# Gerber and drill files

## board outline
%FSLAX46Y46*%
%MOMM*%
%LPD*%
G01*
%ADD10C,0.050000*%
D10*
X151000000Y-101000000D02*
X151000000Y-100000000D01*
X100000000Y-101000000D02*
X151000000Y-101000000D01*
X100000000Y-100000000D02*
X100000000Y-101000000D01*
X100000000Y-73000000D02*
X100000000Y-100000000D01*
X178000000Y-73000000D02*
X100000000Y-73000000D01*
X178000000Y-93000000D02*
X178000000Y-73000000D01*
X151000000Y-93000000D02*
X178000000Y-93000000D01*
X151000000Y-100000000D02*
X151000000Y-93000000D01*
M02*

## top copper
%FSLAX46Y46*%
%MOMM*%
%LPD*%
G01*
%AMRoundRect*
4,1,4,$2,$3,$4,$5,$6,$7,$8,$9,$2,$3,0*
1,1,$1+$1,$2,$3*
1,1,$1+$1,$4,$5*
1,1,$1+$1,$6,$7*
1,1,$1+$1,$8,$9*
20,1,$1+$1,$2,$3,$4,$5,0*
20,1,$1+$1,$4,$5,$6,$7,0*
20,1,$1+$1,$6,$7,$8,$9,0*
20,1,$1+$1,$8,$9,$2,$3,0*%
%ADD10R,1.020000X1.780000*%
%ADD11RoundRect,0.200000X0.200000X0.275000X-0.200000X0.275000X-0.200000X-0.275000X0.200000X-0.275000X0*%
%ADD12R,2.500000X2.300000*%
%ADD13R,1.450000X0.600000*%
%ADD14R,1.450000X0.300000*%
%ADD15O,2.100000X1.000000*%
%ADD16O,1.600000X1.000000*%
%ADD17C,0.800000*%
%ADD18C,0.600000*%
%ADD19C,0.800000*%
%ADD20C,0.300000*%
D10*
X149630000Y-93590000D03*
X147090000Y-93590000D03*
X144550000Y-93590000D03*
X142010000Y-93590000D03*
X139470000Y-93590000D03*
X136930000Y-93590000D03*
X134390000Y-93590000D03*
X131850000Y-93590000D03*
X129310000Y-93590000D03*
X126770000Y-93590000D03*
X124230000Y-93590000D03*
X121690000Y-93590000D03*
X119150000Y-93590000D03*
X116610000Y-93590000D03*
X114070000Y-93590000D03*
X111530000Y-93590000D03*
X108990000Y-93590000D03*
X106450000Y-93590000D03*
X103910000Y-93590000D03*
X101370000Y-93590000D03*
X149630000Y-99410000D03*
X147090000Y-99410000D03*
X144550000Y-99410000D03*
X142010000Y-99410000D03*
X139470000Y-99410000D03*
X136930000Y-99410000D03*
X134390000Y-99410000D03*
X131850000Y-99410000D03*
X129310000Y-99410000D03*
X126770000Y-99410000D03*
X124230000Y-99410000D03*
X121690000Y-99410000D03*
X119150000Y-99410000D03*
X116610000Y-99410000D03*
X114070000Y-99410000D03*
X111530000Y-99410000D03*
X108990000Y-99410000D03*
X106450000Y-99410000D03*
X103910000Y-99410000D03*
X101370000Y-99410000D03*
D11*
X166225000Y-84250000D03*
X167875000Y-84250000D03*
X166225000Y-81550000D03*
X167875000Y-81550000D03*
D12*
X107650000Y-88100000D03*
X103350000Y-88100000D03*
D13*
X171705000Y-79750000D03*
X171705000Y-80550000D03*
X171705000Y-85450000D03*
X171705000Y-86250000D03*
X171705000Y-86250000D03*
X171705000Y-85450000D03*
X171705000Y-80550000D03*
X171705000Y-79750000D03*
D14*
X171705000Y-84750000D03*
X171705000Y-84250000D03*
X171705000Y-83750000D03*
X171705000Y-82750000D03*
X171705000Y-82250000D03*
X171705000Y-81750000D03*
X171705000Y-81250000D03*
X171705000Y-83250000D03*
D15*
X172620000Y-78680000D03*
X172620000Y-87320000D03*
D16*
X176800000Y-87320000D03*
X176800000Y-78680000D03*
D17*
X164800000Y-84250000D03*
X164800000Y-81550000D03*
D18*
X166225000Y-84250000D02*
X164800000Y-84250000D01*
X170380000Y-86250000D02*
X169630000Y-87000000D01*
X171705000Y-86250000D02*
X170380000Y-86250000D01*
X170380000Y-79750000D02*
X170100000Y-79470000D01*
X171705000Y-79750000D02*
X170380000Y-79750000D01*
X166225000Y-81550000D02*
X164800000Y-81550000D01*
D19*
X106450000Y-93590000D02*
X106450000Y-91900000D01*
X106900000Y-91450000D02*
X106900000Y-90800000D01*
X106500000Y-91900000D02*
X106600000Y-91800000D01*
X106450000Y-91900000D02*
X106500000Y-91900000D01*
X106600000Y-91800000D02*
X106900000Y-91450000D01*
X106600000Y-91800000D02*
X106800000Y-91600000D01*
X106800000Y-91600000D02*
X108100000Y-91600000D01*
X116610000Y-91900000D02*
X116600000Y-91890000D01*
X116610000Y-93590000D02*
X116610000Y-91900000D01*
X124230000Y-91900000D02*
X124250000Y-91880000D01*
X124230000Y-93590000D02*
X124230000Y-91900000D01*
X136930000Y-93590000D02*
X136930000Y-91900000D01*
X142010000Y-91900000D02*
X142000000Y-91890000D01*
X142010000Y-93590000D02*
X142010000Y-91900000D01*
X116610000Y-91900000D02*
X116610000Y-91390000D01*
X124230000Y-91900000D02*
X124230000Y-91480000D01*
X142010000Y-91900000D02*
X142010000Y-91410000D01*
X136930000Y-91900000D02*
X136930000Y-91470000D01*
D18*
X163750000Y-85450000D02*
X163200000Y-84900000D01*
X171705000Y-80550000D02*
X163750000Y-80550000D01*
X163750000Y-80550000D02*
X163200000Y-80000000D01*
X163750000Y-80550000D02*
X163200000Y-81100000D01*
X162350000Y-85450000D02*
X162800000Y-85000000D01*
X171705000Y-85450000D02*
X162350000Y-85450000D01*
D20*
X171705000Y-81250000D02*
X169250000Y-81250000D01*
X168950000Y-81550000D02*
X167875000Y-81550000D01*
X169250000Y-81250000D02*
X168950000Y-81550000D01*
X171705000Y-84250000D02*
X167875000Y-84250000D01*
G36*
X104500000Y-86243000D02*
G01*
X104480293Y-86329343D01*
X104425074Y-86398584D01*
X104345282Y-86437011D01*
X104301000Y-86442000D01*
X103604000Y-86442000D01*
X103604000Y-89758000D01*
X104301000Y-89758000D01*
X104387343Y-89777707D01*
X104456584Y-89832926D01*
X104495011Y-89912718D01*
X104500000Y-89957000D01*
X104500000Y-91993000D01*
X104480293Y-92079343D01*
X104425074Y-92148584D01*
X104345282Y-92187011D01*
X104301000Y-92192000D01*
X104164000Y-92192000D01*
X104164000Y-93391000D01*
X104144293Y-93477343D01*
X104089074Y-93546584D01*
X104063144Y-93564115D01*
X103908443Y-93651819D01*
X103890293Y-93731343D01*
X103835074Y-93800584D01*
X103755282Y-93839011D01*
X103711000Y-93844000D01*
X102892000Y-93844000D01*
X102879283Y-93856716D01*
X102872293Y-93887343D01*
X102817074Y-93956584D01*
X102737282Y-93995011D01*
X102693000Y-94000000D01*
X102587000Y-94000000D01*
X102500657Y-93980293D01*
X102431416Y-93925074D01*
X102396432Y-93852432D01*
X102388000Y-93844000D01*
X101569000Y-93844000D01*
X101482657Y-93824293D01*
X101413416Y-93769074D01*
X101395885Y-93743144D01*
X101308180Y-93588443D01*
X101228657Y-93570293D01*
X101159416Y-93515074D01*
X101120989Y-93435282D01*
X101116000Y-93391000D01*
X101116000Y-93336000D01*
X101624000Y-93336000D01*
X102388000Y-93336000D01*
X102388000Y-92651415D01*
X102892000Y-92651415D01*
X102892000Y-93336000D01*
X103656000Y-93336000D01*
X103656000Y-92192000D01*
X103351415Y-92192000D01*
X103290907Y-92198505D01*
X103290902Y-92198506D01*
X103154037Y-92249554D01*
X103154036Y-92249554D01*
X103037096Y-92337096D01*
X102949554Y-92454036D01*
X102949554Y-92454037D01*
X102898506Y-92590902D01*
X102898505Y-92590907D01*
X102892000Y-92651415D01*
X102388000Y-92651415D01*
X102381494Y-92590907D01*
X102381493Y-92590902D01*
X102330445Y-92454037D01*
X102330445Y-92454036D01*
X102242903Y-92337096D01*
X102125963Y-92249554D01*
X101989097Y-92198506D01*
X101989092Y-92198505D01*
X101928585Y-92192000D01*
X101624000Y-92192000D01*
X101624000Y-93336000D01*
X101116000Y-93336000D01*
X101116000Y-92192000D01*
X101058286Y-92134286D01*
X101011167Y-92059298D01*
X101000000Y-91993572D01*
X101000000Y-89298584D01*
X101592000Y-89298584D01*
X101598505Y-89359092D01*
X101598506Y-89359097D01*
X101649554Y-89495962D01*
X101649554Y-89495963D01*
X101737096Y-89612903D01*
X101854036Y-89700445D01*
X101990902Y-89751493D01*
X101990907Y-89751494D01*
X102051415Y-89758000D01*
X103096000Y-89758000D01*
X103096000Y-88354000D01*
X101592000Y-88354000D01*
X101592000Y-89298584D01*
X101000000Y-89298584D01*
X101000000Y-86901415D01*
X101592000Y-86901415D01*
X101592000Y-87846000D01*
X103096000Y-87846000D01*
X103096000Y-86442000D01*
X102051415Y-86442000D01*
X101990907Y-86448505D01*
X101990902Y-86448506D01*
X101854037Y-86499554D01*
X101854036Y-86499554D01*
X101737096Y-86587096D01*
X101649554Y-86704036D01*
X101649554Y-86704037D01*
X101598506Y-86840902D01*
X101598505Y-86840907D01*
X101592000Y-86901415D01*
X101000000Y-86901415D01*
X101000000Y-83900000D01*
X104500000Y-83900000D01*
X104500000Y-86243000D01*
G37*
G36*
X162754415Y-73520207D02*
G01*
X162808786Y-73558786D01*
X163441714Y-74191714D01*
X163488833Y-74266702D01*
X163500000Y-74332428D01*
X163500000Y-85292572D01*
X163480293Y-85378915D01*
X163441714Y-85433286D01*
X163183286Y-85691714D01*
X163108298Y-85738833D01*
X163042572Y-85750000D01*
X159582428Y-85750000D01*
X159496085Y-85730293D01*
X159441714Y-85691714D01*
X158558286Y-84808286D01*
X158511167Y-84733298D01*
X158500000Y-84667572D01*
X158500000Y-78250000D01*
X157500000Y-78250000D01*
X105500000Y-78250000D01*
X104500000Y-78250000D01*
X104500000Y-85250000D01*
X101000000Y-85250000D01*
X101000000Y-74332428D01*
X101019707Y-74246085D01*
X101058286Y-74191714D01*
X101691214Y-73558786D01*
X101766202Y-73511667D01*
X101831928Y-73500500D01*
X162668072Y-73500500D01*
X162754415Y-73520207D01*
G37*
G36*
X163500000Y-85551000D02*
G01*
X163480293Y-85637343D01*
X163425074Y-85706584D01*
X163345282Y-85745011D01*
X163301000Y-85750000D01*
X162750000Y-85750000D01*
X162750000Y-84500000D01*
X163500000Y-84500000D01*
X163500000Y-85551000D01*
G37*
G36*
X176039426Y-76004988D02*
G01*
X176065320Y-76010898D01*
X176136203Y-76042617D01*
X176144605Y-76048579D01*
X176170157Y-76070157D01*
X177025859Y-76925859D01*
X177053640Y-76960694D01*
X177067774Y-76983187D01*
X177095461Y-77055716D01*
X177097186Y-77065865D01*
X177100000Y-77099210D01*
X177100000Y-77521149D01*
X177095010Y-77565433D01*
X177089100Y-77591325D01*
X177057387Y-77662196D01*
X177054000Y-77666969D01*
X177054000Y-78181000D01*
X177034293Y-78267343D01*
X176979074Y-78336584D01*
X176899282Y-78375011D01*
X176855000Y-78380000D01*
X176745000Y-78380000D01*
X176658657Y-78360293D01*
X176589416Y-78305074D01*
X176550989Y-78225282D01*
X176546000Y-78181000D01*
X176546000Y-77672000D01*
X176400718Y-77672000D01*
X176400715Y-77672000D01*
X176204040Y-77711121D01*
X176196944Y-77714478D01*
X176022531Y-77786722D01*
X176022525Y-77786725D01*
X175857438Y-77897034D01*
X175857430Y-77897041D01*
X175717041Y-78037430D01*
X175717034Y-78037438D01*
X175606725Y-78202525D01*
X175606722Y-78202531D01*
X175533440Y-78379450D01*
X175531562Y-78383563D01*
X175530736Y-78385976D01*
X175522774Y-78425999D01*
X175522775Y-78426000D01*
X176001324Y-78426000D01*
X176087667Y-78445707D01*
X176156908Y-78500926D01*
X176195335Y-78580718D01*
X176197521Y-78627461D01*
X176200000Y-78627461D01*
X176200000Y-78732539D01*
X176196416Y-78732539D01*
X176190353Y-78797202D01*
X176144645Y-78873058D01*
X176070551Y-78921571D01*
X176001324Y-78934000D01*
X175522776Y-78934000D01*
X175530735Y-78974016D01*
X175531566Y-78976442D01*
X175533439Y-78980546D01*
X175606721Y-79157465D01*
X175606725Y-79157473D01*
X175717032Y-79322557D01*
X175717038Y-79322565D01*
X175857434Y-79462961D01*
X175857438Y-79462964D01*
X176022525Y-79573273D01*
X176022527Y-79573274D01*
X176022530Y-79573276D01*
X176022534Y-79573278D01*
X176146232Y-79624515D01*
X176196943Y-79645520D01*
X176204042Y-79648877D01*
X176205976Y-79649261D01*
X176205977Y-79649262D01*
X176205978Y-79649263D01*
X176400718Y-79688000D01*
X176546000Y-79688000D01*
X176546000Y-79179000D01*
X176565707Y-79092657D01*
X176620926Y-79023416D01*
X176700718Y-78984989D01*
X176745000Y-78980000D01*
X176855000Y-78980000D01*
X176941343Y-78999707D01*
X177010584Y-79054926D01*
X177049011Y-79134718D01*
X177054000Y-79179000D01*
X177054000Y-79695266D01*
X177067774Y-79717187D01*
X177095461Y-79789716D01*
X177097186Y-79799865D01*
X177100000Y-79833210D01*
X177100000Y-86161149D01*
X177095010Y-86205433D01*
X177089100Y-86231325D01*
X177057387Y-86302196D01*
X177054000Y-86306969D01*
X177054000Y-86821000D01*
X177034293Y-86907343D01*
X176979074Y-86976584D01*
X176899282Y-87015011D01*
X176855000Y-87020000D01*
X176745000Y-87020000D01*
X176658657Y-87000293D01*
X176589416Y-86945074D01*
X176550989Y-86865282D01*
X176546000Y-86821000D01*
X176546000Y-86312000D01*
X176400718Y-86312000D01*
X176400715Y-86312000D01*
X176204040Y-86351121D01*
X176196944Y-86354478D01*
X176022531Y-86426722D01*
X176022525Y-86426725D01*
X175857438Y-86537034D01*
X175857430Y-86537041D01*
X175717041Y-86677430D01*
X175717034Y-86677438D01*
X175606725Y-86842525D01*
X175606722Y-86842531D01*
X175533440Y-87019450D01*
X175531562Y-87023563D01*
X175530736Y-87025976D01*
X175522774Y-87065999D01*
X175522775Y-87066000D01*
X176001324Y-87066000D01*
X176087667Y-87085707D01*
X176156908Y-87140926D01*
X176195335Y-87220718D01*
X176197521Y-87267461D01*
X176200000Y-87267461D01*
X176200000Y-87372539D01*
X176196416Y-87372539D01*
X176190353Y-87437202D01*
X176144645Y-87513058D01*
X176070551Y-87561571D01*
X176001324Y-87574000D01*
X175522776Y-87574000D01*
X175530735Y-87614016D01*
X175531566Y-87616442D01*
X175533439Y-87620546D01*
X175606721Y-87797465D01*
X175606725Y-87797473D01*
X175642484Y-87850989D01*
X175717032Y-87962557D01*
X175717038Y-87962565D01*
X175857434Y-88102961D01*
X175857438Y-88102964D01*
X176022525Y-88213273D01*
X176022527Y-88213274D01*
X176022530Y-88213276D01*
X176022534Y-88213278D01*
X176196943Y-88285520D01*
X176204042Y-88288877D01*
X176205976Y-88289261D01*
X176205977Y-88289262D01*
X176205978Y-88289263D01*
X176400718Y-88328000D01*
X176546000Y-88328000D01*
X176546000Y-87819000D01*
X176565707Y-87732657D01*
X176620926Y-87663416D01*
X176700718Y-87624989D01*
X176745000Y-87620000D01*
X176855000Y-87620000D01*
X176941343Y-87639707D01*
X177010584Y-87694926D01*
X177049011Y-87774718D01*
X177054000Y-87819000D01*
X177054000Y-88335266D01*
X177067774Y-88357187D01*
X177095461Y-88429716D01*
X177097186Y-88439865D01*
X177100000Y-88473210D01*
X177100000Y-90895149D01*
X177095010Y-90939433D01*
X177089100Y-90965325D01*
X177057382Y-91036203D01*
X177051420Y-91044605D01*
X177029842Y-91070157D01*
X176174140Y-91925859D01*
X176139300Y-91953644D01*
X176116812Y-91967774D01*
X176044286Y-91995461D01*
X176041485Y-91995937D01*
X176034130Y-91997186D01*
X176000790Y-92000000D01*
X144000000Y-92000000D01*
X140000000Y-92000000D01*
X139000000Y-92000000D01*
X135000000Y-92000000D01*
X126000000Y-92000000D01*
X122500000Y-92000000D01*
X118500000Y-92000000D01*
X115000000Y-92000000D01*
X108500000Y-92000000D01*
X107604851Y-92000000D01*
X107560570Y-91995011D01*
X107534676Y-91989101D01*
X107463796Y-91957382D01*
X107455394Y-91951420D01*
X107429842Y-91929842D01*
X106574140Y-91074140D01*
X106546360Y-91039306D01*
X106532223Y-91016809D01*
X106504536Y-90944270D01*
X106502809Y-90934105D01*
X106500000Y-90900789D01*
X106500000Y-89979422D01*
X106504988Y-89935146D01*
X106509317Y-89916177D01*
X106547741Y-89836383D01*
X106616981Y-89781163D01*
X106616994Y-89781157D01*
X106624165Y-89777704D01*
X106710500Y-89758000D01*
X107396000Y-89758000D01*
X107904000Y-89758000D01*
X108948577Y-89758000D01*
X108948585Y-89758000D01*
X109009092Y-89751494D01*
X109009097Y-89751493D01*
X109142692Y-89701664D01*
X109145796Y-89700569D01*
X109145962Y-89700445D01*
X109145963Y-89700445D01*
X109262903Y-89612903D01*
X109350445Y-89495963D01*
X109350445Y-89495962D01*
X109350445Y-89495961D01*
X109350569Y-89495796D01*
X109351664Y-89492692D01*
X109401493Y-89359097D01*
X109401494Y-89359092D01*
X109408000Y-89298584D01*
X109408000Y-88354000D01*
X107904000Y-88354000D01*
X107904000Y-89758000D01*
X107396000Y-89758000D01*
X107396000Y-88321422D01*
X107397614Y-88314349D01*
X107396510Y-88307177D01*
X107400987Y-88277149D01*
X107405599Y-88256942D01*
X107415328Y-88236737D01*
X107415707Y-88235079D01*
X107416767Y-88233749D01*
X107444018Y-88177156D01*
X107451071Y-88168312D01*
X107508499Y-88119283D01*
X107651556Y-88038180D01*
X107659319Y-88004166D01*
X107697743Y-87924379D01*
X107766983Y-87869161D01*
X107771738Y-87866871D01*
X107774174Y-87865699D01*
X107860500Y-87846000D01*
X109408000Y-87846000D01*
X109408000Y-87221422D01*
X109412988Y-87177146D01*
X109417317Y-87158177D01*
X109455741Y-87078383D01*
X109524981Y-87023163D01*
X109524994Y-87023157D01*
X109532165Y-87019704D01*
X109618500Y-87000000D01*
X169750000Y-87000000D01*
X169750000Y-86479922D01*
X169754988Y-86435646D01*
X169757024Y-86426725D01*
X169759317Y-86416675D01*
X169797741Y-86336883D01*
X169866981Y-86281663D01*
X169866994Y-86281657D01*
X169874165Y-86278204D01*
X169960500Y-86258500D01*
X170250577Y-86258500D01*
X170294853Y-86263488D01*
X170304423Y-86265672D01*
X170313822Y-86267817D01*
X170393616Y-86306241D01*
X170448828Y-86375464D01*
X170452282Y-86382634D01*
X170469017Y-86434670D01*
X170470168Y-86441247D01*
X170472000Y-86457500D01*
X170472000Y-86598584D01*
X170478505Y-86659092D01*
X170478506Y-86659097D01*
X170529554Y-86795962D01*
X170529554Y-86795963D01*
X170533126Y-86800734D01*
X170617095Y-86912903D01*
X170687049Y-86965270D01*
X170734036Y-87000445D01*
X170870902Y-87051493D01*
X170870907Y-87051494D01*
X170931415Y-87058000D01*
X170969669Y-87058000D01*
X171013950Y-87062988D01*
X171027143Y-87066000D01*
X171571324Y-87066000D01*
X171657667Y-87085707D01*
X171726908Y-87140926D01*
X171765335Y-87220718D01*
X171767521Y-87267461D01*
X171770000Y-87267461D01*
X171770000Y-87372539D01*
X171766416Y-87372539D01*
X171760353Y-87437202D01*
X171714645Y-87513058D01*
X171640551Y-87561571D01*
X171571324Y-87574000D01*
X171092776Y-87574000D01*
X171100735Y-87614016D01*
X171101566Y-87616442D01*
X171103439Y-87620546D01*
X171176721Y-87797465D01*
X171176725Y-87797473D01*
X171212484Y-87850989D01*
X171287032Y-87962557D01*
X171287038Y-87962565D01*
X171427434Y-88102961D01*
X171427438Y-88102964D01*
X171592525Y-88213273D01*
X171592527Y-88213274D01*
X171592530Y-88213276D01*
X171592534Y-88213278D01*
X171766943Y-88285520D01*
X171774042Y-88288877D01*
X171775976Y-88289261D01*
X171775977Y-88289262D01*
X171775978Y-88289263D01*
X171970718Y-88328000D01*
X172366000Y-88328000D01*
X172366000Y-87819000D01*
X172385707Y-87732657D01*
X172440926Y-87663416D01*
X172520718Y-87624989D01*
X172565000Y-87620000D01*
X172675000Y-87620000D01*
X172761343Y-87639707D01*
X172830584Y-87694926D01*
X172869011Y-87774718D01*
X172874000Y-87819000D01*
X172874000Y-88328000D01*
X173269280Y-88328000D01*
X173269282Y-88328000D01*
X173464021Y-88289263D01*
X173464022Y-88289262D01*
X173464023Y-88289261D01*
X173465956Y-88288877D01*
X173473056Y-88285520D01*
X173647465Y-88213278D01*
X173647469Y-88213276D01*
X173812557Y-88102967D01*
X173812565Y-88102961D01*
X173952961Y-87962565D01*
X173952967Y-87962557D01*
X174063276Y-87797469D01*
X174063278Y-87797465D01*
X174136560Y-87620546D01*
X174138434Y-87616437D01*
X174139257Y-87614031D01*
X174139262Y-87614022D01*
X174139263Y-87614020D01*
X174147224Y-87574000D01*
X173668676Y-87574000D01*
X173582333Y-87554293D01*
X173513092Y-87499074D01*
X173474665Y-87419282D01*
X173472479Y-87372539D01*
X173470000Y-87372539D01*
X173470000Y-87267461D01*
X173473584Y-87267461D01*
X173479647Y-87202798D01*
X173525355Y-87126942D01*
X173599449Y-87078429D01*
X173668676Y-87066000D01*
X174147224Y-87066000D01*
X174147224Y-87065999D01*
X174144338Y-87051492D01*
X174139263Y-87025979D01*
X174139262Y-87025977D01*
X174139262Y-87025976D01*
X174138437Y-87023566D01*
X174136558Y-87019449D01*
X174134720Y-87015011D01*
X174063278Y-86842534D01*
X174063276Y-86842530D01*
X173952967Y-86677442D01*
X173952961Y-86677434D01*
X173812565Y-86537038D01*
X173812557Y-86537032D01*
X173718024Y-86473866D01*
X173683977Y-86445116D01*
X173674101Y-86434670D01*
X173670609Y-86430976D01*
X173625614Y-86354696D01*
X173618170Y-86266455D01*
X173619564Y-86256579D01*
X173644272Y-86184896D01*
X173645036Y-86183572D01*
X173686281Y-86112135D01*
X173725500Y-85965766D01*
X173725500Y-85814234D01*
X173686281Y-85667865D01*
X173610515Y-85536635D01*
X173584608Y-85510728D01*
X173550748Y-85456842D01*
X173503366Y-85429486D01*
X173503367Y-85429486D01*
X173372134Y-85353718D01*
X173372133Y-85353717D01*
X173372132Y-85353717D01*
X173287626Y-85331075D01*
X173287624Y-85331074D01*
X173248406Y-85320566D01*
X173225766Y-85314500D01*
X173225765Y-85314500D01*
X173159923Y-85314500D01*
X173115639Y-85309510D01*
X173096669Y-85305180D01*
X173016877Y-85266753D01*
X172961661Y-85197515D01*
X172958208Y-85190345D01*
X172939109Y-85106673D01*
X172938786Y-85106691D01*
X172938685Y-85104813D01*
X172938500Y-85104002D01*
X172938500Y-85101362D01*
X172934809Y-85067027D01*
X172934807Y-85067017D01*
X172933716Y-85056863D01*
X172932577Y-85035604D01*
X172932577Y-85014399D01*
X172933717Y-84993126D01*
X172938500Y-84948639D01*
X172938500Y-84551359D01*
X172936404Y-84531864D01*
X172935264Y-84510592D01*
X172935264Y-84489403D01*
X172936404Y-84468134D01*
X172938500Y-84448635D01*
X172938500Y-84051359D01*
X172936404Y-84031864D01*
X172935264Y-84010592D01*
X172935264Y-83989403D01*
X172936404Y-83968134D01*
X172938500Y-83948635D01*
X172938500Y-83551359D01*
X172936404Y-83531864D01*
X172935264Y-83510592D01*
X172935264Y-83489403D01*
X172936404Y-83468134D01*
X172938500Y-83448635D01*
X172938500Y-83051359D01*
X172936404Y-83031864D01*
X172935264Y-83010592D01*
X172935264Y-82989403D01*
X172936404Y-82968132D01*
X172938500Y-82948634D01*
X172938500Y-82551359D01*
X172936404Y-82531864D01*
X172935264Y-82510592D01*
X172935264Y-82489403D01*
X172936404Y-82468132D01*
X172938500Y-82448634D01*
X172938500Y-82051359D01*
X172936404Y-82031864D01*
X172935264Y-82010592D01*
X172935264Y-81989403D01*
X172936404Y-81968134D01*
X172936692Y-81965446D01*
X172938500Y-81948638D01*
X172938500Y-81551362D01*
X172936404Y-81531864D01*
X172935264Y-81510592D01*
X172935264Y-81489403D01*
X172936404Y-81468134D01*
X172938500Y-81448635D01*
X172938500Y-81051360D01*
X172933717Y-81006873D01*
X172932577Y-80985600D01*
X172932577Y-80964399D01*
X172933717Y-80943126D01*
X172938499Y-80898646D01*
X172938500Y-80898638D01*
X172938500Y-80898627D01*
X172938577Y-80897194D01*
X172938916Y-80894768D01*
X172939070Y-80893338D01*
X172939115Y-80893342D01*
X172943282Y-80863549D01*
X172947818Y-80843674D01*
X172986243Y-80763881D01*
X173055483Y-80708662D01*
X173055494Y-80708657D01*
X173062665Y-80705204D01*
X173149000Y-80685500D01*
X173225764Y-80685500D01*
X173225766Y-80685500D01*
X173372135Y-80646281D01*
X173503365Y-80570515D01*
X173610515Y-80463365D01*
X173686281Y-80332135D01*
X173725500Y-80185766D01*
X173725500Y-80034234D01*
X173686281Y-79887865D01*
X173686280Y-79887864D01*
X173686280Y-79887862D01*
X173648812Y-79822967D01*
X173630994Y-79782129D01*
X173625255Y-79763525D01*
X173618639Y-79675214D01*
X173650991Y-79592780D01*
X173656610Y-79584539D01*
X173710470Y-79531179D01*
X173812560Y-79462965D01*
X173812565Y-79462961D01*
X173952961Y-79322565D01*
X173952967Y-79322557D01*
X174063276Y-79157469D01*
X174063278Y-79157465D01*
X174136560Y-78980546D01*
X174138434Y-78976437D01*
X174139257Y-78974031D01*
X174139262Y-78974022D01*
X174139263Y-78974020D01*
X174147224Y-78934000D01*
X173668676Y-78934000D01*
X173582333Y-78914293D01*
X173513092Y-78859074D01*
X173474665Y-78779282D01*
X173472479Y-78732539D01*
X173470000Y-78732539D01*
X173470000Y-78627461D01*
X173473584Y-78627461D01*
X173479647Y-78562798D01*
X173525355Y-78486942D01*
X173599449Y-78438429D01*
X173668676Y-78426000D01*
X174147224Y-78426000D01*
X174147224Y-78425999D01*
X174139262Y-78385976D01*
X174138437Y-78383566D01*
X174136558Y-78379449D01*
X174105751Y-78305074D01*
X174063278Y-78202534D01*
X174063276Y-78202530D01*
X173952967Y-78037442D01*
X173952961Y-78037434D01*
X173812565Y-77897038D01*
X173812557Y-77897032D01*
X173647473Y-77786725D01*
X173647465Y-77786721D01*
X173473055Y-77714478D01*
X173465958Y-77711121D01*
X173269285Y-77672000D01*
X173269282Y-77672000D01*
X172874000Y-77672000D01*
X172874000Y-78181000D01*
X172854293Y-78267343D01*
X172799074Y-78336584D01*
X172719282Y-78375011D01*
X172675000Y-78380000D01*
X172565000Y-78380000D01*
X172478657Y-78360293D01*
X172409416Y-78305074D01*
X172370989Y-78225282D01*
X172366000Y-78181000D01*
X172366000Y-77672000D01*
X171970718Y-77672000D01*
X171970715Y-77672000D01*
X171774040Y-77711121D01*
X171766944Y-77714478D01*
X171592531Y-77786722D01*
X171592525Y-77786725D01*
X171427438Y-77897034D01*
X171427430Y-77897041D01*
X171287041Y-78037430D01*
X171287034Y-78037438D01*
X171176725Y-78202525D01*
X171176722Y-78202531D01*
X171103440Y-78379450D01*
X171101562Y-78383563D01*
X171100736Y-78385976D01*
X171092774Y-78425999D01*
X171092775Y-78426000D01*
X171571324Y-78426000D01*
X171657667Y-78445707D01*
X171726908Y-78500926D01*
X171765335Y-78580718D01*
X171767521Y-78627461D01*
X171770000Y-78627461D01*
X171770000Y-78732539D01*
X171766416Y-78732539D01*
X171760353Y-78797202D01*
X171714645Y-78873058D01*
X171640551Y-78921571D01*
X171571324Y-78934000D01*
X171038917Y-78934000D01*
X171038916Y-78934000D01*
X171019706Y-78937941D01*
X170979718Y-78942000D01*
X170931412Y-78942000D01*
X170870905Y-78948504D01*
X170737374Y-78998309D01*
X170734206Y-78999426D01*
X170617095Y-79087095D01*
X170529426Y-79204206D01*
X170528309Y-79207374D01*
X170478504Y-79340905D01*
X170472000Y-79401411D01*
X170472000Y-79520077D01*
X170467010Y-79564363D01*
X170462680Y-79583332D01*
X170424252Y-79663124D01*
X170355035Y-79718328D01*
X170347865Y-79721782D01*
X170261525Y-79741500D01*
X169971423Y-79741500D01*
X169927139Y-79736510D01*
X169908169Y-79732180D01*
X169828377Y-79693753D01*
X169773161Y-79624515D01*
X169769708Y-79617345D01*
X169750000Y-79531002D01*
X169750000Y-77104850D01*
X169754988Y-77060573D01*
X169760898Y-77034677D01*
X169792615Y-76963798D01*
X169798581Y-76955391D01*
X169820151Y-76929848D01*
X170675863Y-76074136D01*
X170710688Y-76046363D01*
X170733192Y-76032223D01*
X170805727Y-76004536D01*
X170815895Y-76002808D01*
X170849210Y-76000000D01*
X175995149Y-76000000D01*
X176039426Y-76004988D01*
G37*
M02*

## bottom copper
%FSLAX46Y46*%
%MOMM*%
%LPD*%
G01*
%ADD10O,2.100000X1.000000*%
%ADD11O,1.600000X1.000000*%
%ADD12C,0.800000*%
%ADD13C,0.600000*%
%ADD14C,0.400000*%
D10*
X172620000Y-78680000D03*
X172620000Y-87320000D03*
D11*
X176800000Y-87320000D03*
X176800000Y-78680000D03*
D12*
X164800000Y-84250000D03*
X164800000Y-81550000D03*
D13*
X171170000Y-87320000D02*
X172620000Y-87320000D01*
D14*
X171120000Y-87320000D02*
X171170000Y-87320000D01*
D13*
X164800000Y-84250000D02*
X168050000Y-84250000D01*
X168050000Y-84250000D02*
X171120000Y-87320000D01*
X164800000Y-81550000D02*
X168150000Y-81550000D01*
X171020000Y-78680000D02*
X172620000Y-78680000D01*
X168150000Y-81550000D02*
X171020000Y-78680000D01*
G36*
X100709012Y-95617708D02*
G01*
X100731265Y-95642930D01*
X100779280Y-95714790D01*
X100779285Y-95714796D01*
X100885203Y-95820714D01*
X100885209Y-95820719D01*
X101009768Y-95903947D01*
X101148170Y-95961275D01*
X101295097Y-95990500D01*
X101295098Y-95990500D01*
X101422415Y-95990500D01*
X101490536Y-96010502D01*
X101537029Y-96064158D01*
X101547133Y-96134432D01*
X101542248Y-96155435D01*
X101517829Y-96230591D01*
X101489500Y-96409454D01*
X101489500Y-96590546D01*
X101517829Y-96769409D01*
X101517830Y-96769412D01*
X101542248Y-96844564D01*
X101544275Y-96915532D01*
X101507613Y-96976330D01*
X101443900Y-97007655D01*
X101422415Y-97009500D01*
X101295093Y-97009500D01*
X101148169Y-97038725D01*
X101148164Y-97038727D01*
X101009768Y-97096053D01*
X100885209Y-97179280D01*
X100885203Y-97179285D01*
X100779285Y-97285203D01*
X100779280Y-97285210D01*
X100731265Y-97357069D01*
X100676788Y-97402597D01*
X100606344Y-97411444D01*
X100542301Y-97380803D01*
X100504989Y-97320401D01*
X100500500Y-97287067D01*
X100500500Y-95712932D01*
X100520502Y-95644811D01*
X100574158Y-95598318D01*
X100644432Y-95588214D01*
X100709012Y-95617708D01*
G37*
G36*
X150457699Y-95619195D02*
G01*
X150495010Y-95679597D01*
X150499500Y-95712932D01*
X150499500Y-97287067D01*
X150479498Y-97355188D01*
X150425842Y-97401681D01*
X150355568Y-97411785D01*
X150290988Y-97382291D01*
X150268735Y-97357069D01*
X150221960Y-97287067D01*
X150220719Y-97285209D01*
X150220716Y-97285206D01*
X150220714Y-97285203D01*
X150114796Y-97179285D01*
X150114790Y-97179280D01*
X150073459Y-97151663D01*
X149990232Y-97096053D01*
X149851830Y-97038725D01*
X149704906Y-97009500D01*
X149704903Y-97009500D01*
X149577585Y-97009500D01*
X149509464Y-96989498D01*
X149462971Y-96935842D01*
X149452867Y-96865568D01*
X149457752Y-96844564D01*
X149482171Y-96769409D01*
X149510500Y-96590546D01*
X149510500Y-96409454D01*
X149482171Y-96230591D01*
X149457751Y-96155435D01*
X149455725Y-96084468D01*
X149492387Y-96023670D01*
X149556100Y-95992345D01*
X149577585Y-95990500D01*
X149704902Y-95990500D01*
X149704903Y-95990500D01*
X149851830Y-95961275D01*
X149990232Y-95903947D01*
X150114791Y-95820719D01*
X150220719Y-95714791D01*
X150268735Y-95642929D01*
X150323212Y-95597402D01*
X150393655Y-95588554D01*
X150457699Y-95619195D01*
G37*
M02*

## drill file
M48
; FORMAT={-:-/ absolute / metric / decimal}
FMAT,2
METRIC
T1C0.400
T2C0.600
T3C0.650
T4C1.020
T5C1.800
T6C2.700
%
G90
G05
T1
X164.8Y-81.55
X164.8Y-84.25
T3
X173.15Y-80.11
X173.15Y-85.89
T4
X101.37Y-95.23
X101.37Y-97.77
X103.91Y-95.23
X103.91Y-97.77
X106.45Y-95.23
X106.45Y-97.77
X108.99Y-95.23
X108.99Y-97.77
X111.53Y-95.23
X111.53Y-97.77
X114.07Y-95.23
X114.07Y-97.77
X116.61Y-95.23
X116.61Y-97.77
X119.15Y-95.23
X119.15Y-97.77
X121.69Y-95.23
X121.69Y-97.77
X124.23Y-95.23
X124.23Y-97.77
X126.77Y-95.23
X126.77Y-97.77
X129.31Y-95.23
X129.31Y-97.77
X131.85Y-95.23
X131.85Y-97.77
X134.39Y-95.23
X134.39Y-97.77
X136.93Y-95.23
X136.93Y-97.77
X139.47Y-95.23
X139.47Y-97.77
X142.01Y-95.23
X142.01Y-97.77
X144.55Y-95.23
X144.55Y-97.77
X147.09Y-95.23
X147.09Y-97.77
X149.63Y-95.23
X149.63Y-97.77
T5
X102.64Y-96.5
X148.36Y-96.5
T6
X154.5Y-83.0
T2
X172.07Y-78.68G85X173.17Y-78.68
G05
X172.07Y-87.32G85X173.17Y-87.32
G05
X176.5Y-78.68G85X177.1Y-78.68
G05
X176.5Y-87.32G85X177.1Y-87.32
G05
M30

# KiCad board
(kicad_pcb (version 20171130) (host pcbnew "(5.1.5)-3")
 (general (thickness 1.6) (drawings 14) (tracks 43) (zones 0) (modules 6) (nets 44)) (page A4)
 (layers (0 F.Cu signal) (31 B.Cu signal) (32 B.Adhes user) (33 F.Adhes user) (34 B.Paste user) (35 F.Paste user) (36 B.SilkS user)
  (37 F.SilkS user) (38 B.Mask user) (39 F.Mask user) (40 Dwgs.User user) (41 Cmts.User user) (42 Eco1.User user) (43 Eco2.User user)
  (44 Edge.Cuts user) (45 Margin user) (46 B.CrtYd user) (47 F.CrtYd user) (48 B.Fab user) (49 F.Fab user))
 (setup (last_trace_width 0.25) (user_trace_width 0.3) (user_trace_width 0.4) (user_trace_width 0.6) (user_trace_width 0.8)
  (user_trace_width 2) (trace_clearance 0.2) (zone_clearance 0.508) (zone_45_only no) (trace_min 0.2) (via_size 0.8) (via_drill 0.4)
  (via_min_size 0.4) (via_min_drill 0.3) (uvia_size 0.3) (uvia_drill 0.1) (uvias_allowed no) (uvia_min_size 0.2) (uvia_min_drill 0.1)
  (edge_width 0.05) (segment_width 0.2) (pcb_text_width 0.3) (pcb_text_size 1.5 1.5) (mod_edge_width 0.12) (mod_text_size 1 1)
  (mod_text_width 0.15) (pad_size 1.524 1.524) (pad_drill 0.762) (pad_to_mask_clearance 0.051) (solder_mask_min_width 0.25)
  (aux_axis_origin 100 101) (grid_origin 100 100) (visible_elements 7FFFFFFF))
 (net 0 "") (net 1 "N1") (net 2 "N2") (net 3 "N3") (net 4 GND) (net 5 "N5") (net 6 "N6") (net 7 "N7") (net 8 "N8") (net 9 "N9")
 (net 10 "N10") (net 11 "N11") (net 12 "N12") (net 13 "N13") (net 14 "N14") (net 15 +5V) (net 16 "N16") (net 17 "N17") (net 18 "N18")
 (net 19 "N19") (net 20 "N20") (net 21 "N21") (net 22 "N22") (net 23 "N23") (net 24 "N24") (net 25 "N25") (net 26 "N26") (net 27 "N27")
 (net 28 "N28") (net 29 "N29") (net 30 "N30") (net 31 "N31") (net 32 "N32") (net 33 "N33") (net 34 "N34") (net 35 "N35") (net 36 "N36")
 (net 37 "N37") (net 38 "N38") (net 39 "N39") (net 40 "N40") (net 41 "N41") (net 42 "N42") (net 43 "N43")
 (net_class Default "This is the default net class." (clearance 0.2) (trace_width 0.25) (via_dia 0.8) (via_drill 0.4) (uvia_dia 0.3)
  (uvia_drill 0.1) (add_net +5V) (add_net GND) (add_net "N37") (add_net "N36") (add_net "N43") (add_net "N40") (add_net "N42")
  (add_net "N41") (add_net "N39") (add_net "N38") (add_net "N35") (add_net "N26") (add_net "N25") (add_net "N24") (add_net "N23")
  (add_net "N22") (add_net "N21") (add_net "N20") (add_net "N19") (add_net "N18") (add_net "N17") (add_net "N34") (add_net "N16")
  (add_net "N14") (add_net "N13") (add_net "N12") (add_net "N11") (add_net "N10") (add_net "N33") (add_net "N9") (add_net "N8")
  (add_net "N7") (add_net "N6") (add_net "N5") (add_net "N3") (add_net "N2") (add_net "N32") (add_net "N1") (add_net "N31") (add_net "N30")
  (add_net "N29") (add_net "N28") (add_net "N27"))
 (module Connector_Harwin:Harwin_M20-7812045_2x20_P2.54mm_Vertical (layer F.Cu) (at 125.5 96.5 90)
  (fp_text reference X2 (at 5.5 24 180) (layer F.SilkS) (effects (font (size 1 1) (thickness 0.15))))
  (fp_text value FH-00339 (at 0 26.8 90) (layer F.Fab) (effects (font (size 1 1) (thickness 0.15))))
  (pad 40 smd rect (at 2.91 24.13 90) (size 1.78 1.02) (layers F.Cu F.Paste F.Mask) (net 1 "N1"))
  (pad 39 smd rect (at 2.91 21.59 90) (size 1.78 1.02) (layers F.Cu F.Paste F.Mask) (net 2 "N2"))
  (pad 38 smd rect (at 2.91 19.05 90) (size 1.78 1.02) (layers F.Cu F.Paste F.Mask) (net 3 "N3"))
  (pad 37 smd rect (at 2.91 16.51 90) (size 1.78 1.02) (layers F.Cu F.Paste F.Mask) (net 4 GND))
  (pad 36 smd rect (at 2.91 13.97 90) (size 1.78 1.02) (layers F.Cu F.Paste F.Mask) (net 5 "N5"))
  (pad 35 smd rect (at 2.91 11.43 90) (size 1.78 1.02) (layers F.Cu F.Paste F.Mask) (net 4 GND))
  (pad 34 smd rect (at 2.91 8.89 90) (size 1.78 1.02) (layers F.Cu F.Paste F.Mask) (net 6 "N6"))
  (pad 33 smd rect (at 2.91 6.35 90) (size 1.78 1.02) (layers F.Cu F.Paste F.Mask) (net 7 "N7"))
  (pad 32 smd rect (at 2.91 3.81 90) (size 1.78 1.02) (layers F.Cu F.Paste F.Mask) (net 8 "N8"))
  (pad 31 smd rect (at 2.91 1.27 90) (size 1.78 1.02) (layers F.Cu F.Paste F.Mask) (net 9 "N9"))
  (pad 30 smd rect (at 2.91 -1.27 90) (size 1.78 1.02) (layers F.Cu F.Paste F.Mask) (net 4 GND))
  (pad 29 smd rect (at 2.91 -3.81 90) (size 1.78 1.02) (layers F.Cu F.Paste F.Mask) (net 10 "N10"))
  (pad 28 smd rect (at 2.91 -6.35 90) (size 1.78 1.02) (layers F.Cu F.Paste F.Mask) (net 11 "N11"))
  (pad 27 smd rect (at 2.91 -8.89 90) (size 1.78 1.02) (layers F.Cu F.Paste F.Mask) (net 4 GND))
  (pad 26 smd rect (at 2.91 -11.43 90) (size 1.78 1.02) (layers F.Cu F.Paste F.Mask) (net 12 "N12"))
  (pad 25 smd rect (at 2.91 -13.97 90) (size 1.78 1.02) (layers F.Cu F.Paste F.Mask) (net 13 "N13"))
  (pad 24 smd rect (at 2.91 -16.51 90) (size 1.78 1.02) (layers F.Cu F.Paste F.Mask) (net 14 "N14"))
  (pad 23 smd rect (at 2.91 -19.05 90) (size 1.78 1.02) (layers F.Cu F.Paste F.Mask) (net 4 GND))
  (pad 22 smd rect (at 2.91 -21.59 90) (size 1.78 1.02) (layers F.Cu F.Paste F.Mask) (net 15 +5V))
  (pad 21 smd rect (at 2.91 -24.13 90) (size 1.78 1.02) (layers F.Cu F.Paste F.Mask) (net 15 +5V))
  (pad 20 smd rect (at -2.91 24.13 90) (size 1.78 1.02) (layers F.Cu F.Paste F.Mask) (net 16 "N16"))
  (pad 19 smd rect (at -2.91 21.59 90) (size 1.78 1.02) (layers F.Cu F.Paste F.Mask) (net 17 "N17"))
  (pad 18 smd rect (at -2.91 19.05 90) (size 1.78 1.02) (layers F.Cu F.Paste F.Mask) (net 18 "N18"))
  (pad 17 smd rect (at -2.91 16.51 90) (size 1.78 1.02) (layers F.Cu F.Paste F.Mask) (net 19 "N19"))
  (pad 16 smd rect (at -2.91 13.97 90) (size 1.78 1.02) (layers F.Cu F.Paste F.Mask) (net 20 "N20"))
  (pad 15 smd rect (at -2.91 11.43 90) (size 1.78 1.02) (layers F.Cu F.Paste F.Mask) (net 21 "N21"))
  (pad 14 smd rect (at -2.91 8.89 90) (size 1.78 1.02) (layers F.Cu F.Paste F.Mask) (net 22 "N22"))
  (pad 13 smd rect (at -2.91 6.35 90) (size 1.78 1.02) (layers F.Cu F.Paste F.Mask) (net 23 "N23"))
  (pad 12 smd rect (at -2.91 3.81 90) (size 1.78 1.02) (layers F.Cu F.Paste F.Mask) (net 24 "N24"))
  (pad 11 smd rect (at -2.91 1.27 90) (size 1.78 1.02) (layers F.Cu F.Paste F.Mask) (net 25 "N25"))
  (pad 10 smd rect (at -2.91 -1.27 90) (size 1.78 1.02) (layers F.Cu F.Paste F.Mask) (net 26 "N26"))
  (pad 9 smd rect (at -2.91 -3.81 90) (size 1.78 1.02) (layers F.Cu F.Paste F.Mask) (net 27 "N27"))
  (pad 8 smd rect (at -2.91 -6.35 90) (size 1.78 1.02) (layers F.Cu F.Paste F.Mask) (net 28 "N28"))
  (pad 7 smd rect (at -2.91 -8.89 90) (size 1.78 1.02) (layers F.Cu F.Paste F.Mask) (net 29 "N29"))
  (pad 6 smd rect (at -2.91 -11.43 90) (size 1.78 1.02) (layers F.Cu F.Paste F.Mask) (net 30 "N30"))
  (pad 5 smd rect (at -2.91 -13.97 90) (size 1.78 1.02) (layers F.Cu F.Paste F.Mask) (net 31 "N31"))
  (pad 4 smd rect (at -2.91 -16.51 90) (size 1.78 1.02) (layers F.Cu F.Paste F.Mask) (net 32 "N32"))
  (pad 3 smd rect (at -2.91 -19.05 90) (size 1.78 1.02) (layers F.Cu F.Paste F.Mask) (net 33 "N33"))
  (pad 2 smd rect (at -2.91 -21.59 90) (size 1.78 1.02) (layers F.Cu F.Paste F.Mask) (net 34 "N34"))
  (pad 1 smd rect (at -2.91 -24.13 90) (size 1.78 1.02) (layers F.Cu F.Paste F.Mask) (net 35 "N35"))
  (pad "" np_thru_hole circle (at 1.27 24.13 90) (size 1.02 1.02) (drill 1.02) (layers *.Cu *.Mask))
  (pad "" np_thru_hole circle (at 1.27 21.59 90) (size 1.02 1.02) (drill 1.02) (layers *.Cu *.Mask))
  (pad "" np_thru_hole circle (at 1.27 19.05 90) (size 1.02 1.02) (drill 1.02) (layers *.Cu *.Mask))
  (pad "" np_thru_hole circle (at 1.27 16.51 90) (size 1.02 1.02) (drill 1.02) (layers *.Cu *.Mask))
  (pad "" np_thru_hole circle (at 1.27 13.97 90) (size 1.02 1.02) (drill 1.02) (layers *.Cu *.Mask))
  (pad "" np_thru_hole circle (at 1.27 11.43 90) (size 1.02 1.02) (drill 1.02) (layers *.Cu *.Mask))
  (pad "" np_thru_hole circle (at 1.27 8.89 90) (size 1.02 1.02) (drill 1.02) (layers *.Cu *.Mask))
  (pad "" np_thru_hole circle (at 1.27 6.35 90) (size 1.02 1.02) (drill 1.02) (layers *.Cu *.Mask))
  (pad "" np_thru_hole circle (at 1.27 3.81 90) (size 1.02 1.02) (drill 1.02) (layers *.Cu *.Mask))
  (pad "" np_thru_hole circle (at 1.27 1.27 90) (size 1.02 1.02) (drill 1.02) (layers *.Cu *.Mask))
  (pad "" np_thru_hole circle (at 1.27 -1.27 90) (size 1.02 1.02) (drill 1.02) (layers *.Cu *.Mask))
  (pad "" np_thru_hole circle (at 1.27 -3.81 90) (size 1.02 1.02) (drill 1.02) (layers *.Cu *.Mask))
  (pad "" np_thru_hole circle (at 1.27 -6.35 90) (size 1.02 1.02) (drill 1.02) (layers *.Cu *.Mask))
  (pad "" np_thru_hole circle (at 1.27 -8.89 90) (size 1.02 1.02) (drill 1.02) (layers *.Cu *.Mask))
  (pad "" np_thru_hole circle (at 1.27 -11.43 90) (size 1.02 1.02) (drill 1.02) (layers *.Cu *.Mask))
  (pad "" np_thru_hole circle (at 1.27 -13.97 90) (size 1.02 1.02) (drill 1.02) (layers *.Cu *.Mask))
  (pad "" np_thru_hole circle (at 1.27 -16.51 90) (size 1.02 1.02) (drill 1.02) (layers *.Cu *.Mask))
  (pad "" np_thru_hole circle (at 1.27 -19.05 90) (size 1.02 1.02) (drill 1.02) (layers *.Cu *.Mask))
  (pad "" np_thru_hole circle (at 1.27 -21.59 90) (size 1.02 1.02) (drill 1.02) (layers *.Cu *.Mask))
  (pad "" np_thru_hole circle (at 1.27 -24.13 90) (size 1.02 1.02) (drill 1.02) (layers *.Cu *.Mask))
  (pad "" np_thru_hole circle (at -1.27 24.13 90) (size 1.02 1.02) (drill 1.02) (layers *.Cu *.Mask))
  (pad "" np_thru_hole circle (at -1.27 21.59 90) (size 1.02 1.02) (drill 1.02) (layers *.Cu *.Mask))
  (pad "" np_thru_hole circle (at -1.27 19.05 90) (size 1.02 1.02) (drill 1.02) (layers *.Cu *.Mask))
  (pad "" np_thru_hole circle (at -1.27 16.51 90) (size 1.02 1.02) (drill 1.02) (layers *.Cu *.Mask))
  (pad "" np_thru_hole circle (at -1.27 13.97 90) (size 1.02 1.02) (drill 1.02) (layers *.Cu *.Mask))
  (pad "" np_thru_hole circle (at -1.27 11.43 90) (size 1.02 1.02) (drill 1.02) (layers *.Cu *.Mask))
  (pad "" np_thru_hole circle (at -1.27 8.89 90) (size 1.02 1.02) (drill 1.02) (layers *.Cu *.Mask))
  (pad "" np_thru_hole circle (at -1.27 6.35 90) (size 1.02 1.02) (drill 1.02) (layers *.Cu *.Mask))
  (pad "" np_thru_hole circle (at -1.27 3.81 90) (size 1.02 1.02) (drill 1.02) (layers *.Cu *.Mask))
  (pad "" np_thru_hole circle (at -1.27 1.27 90) (size 1.02 1.02) (drill 1.02) (layers *.Cu *.Mask))
  (pad "" np_thru_hole circle (at -1.27 -1.27 90) (size 1.02 1.02) (drill 1.02) (layers *.Cu *.Mask))
  (pad "" np_thru_hole circle (at -1.27 -3.81 90) (size 1.02 1.02) (drill 1.02) (layers *.Cu *.Mask))
  (pad "" np_thru_hole circle (at -1.27 -6.35 90) (size 1.02 1.02) (drill 1.02) (layers *.Cu *.Mask))
  (pad "" np_thru_hole circle (at -1.27 -8.89 90) (size 1.02 1.02) (drill 1.02) (layers *.Cu *.Mask))
  (pad "" np_thru_hole circle (at -1.27 -11.43 90) (size 1.02 1.02) (drill 1.02) (layers *.Cu *.Mask))
  (pad "" np_thru_hole circle (at -1.27 -13.97 90) (size 1.02 1.02) (drill 1.02) (layers *.Cu *.Mask))
  (pad "" np_thru_hole circle (at -1.27 -16.51 90) (size 1.02 1.02) (drill 1.02) (layers *.Cu *.Mask))
  (pad "" np_thru_hole circle (at -1.27 -19.05 90) (size 1.02 1.02) (drill 1.02) (layers *.Cu *.Mask))
  (pad "" np_thru_hole circle (at -1.27 -21.59 90) (size 1.02 1.02) (drill 1.02) (layers *.Cu *.Mask))
  (pad "" np_thru_hole circle (at -1.27 -24.13 90) (size 1.02 1.02) (drill 1.02) (layers *.Cu *.Mask))
  (pad "" np_thru_hole circle (at 0 22.86 90) (size 1.8 1.8) (drill 1.8) (layers *.Cu *.Mask))
  (pad "" np_thru_hole circle (at 0 -22.86 90) (size 1.8 1.8) (drill 1.8) (layers *.Cu *.Mask)))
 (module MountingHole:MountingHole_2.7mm (layer F.Cu) (at 154.5 83)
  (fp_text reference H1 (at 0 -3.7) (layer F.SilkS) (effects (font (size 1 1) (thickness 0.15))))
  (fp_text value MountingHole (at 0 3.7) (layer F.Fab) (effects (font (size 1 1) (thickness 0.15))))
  (pad 1 np_thru_hole circle (at 0 0) (size 2.7 2.7) (drill 2.7) (layers *.Cu *.Mask)))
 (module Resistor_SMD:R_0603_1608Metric (layer F.Cu) (at 167.05 84.25 180)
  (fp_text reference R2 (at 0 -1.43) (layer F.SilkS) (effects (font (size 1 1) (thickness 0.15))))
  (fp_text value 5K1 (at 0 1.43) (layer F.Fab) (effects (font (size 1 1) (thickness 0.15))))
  (pad 2 smd roundrect (at 0.825 0 180) (size 0.8 0.95) (layers F.Cu F.Paste F.Mask) (roundrect_rratio 0.25) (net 4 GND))
  (pad 1 smd roundrect (at -0.825 0 180) (size 0.8 0.95) (layers F.Cu F.Paste F.Mask) (roundrect_rratio 0.25) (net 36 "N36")))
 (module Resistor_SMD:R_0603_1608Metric (layer F.Cu) (at 167.05 81.55 180)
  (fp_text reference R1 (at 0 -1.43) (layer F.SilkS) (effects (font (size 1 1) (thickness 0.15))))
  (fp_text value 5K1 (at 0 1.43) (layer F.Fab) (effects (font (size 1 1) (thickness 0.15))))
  (pad 2 smd roundrect (at 0.825 0 180) (size 0.8 0.95) (layers F.Cu F.Paste F.Mask) (roundrect_rratio 0.25) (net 4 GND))
  (pad 1 smd roundrect (at -0.825 0 180) (size 0.8 0.95) (layers F.Cu F.Paste F.Mask) (roundrect_rratio 0.25) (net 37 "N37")))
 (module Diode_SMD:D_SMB (layer F.Cu) (at 105.5 88.1)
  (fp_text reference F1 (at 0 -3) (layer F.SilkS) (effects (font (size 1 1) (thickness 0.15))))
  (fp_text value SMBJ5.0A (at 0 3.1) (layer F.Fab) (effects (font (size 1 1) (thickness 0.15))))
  (pad 2 smd rect (at 2.15 0) (size 2.5 2.3) (layers F.Cu F.Paste F.Mask) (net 4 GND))
  (pad 1 smd rect (at -2.15 0) (size 2.5 2.3) (layers F.Cu F.Paste F.Mask) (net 15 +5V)))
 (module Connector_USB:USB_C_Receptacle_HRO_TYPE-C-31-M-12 (layer F.Cu) (at 175.75 83 90)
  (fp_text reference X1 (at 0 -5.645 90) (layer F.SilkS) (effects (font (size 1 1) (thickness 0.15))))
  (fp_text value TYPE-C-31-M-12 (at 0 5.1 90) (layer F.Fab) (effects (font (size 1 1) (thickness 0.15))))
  (pad B1 smd rect (at 3.25 -4.045 90) (size 0.6 1.45) (layers F.Cu F.Paste F.Mask) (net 4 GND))
  (pad A9 smd rect (at 2.45 -4.045 90) (size 0.6 1.45) (layers F.Cu F.Paste F.Mask) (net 15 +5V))
  (pad B9 smd rect (at -2.45 -4.045 90) (size 0.6 1.45) (layers F.Cu F.Paste F.Mask) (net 15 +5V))
  (pad B12 smd rect (at -3.25 -4.045 90) (size 0.6 1.45) (layers F.Cu F.Paste F.Mask) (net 4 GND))
  (pad A1 smd rect (at -3.25 -4.045 90) (size 0.6 1.45) (layers F.Cu F.Paste F.Mask) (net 4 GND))
  (pad A4 smd rect (at -2.45 -4.045 90) (size 0.6 1.45) (layers F.Cu F.Paste F.Mask) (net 15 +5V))
  (pad B4 smd rect (at 2.45 -4.045 90) (size 0.6 1.45) (layers F.Cu F.Paste F.Mask) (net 15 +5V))
  (pad A12 smd rect (at 3.25 -4.045 90) (size 0.6 1.45) (layers F.Cu F.Paste F.Mask) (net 4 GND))
  (pad B8 smd rect (at -1.75 -4.045 90) (size 0.3 1.45) (layers F.Cu F.Paste F.Mask) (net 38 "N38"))
  (pad A5 smd rect (at -1.25 -4.045 90) (size 0.3 1.45) (layers F.Cu F.Paste F.Mask) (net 36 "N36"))
  (pad B7 smd rect (at -0.75 -4.045 90) (size 0.3 1.45) (layers F.Cu F.Paste F.Mask) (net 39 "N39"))
  (pad A7 smd rect (at 0.25 -4.045 90) (size 0.3 1.45) (layers F.Cu F.Paste F.Mask) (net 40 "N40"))
  (pad B6 smd rect (at 0.75 -4.045 90) (size 0.3 1.45) (layers F.Cu F.Paste F.Mask) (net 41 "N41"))
  (pad A8 smd rect (at 1.25 -4.045 90) (size 0.3 1.45) (layers F.Cu F.Paste F.Mask) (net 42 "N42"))
  (pad B5 smd rect (at 1.75 -4.045 90) (size 0.3 1.45) (layers F.Cu F.Paste F.Mask) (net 37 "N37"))
  (pad A6 smd rect (at -0.25 -4.045 90) (size 0.3 1.45) (layers F.Cu F.Paste F.Mask) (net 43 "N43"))
  (pad S1 thru_hole oval (at 4.32 -3.13 90) (size 1 2.1) (drill oval 0.6 1.7) (layers *.Cu *.Mask) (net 4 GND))
  (pad S1 thru_hole oval (at -4.32 -3.13 90) (size 1 2.1) (drill oval 0.6 1.7) (layers *.Cu *.Mask) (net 4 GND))
  (pad "" np_thru_hole circle (at -2.89 -2.6 90) (size 0.65 0.65) (drill 0.65) (layers *.Cu *.Mask))
  (pad S1 thru_hole oval (at -4.32 1.05 90) (size 1 1.6) (drill oval 0.6 1.2) (layers *.Cu *.Mask) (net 4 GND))
  (pad "" np_thru_hole circle (at 2.89 -2.6 90) (size 0.65 0.65) (drill 0.65) (layers *.Cu *.Mask))
  (pad S1 thru_hole oval (at 4.32 1.05 90) (size 1 1.6) (drill oval 0.6 1.2) (layers *.Cu *.Mask) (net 4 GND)))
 (gr_line (start 151 101) (end 151 100) (layer Edge.Cuts) (width 0.05))
 (gr_line (start 100 101) (end 151 101) (layer Edge.Cuts) (width 0.05))
 (gr_line (start 100 100) (end 100 101) (layer Edge.Cuts) (width 0.05))
 (gr_line (start 100 73) (end 100 100) (layer Edge.Cuts) (width 0.05))
 (gr_line (start 178 73) (end 100 73) (layer Edge.Cuts) (width 0.05))
 (gr_line (start 178 93) (end 178 73) (layer Edge.Cuts) (width 0.05))
 (gr_line (start 151 93) (end 178 93) (layer Edge.Cuts) (width 0.05))
 (gr_line (start 151 100) (end 151 93) (layer Edge.Cuts) (width 0.05))
 (via (at 164.8 84.25) (size 0.8) (drill 0.4) (layers F.Cu B.Cu) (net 4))
 (segment (start 166.225 84.25) (end 164.8 84.25) (width 0.6) (layer F.Cu) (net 4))
 (segment (start 171.17 87.32) (end 172.62 87.32) (width 0.6) (layer B.Cu) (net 4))
 (segment (start 171.12 87.32) (end 171.17 87.32) (width 0.4) (layer B.Cu) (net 4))
 (segment (start 164.8 84.25) (end 168.05 84.25) (width 0.6) (layer B.Cu) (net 4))
 (segment (start 168.05 84.25) (end 171.12 87.32) (width 0.6) (layer B.Cu) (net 4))
 (segment (start 170.38 86.25) (end 169.63 87) (width 0.6) (layer F.Cu) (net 4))
 (segment (start 171.705 86.25) (end 170.38 86.25) (width 0.6) (layer F.Cu) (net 4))
 (segment (start 170.38 79.75) (end 170.1 79.47) (width 0.6) (layer F.Cu) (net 4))
 (segment (start 171.705 79.75) (end 170.38 79.75) (width 0.6) (layer F.Cu) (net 4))
 (via (at 164.8 81.55) (size 0.8) (drill 0.4) (layers F.Cu B.Cu) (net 4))
 (segment (start 166.225 81.55) (end 164.8 81.55) (width 0.6) (layer F.Cu) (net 4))
 (segment (start 164.8 81.55) (end 168.15 81.55) (width 0.6) (layer B.Cu) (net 4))
 (segment (start 171.02 78.68) (end 172.62 78.68) (width 0.6) (layer B.Cu) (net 4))
 (segment (start 168.15 81.55) (end 171.02 78.68) (width 0.6) (layer B.Cu) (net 4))
 (segment (start 106.45 93.59) (end 106.45 91.9) (width 0.8) (layer F.Cu) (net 4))
 (segment (start 106.9 91.45) (end 106.9 90.8) (width 0.8) (layer F.Cu) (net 4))
 (segment (start 106.5 91.9) (end 106.6 91.8) (width 0.8) (layer F.Cu) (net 4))
 (segment (start 106.45 91.9) (end 106.5 91.9) (width 0.8) (layer F.Cu) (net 4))
 (segment (start 106.6 91.8) (end 106.9 91.45) (width 0.8) (layer F.Cu) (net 4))
 (segment (start 106.6 91.8) (end 106.8 91.6) (width 0.8) (layer F.Cu) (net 4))
 (segment (start 106.8 91.6) (end 108.1 91.6) (width 0.8) (layer F.Cu) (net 4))
 (segment (start 116.61 91.9) (end 116.6 91.89) (width 0.8) (layer F.Cu) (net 4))
 (segment (start 116.61 93.59) (end 116.61 91.9) (width 0.8) (layer F.Cu) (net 4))
 (segment (start 124.23 91.9) (end 124.25 91.88) (width 0.8) (layer F.Cu) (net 4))
 (segment (start 124.23 93.59) (end 124.23 91.9) (width 0.8) (layer F.Cu) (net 4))
 (segment (start 136.93 93.59) (end 136.93 91.9) (width 0.8) (layer F.Cu) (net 4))
 (segment (start 142.01 91.9) (end 142 91.89) (width 0.8) (layer F.Cu) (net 4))
 (segment (start 142.01 93.59) (end 142.01 91.9) (width 0.8) (layer F.Cu) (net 4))
 (segment (start 116.61 91.9) (end 116.61 91.39) (width 0.8) (layer F.Cu) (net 4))
 (segment (start 124.23 91.9) (end 124.23 91.48) (width 0.8) (layer F.Cu) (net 4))
 (segment (start 142.01 91.9) (end 142.01 91.41) (width 0.8) (layer F.Cu) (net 4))
 (segment (start 136.93 91.9) (end 136.93 91.47) (width 0.8) (layer F.Cu) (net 4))
 (segment (start 163.75 85.45) (end 163.2 84.9) (width 0.6) (layer F.Cu) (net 15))
 (segment (start 171.705 80.55) (end 163.75 80.55) (width 0.6) (layer F.Cu) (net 15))
 (segment (start 163.75 80.55) (end 163.2 80) (width 0.6) (layer F.Cu) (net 15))
 (segment (start 163.75 80.55) (end 163.2 81.1) (width 0.6) (layer F.Cu) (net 15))
 (segment (start 162.35 85.45) (end 162.8 85) (width 0.6) (layer F.Cu) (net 15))
 (segment (start 171.705 85.45) (end 162.35 85.45) (width 0.6) (layer F.Cu) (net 15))
 (segment (start 171.705 81.25) (end 169.25 81.25) (width 0.3) (layer F.Cu) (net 37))
 (segment (start 168.95 81.55) (end 167.875 81.55) (width 0.3) (layer F.Cu) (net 37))
 (segment (start 169.25 81.25) (end 168.95 81.55) (width 0.3) (layer F.Cu) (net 37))
 (segment (start 171.705 84.25) (end 167.875 84.25) (width 0.3) (layer F.Cu) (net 36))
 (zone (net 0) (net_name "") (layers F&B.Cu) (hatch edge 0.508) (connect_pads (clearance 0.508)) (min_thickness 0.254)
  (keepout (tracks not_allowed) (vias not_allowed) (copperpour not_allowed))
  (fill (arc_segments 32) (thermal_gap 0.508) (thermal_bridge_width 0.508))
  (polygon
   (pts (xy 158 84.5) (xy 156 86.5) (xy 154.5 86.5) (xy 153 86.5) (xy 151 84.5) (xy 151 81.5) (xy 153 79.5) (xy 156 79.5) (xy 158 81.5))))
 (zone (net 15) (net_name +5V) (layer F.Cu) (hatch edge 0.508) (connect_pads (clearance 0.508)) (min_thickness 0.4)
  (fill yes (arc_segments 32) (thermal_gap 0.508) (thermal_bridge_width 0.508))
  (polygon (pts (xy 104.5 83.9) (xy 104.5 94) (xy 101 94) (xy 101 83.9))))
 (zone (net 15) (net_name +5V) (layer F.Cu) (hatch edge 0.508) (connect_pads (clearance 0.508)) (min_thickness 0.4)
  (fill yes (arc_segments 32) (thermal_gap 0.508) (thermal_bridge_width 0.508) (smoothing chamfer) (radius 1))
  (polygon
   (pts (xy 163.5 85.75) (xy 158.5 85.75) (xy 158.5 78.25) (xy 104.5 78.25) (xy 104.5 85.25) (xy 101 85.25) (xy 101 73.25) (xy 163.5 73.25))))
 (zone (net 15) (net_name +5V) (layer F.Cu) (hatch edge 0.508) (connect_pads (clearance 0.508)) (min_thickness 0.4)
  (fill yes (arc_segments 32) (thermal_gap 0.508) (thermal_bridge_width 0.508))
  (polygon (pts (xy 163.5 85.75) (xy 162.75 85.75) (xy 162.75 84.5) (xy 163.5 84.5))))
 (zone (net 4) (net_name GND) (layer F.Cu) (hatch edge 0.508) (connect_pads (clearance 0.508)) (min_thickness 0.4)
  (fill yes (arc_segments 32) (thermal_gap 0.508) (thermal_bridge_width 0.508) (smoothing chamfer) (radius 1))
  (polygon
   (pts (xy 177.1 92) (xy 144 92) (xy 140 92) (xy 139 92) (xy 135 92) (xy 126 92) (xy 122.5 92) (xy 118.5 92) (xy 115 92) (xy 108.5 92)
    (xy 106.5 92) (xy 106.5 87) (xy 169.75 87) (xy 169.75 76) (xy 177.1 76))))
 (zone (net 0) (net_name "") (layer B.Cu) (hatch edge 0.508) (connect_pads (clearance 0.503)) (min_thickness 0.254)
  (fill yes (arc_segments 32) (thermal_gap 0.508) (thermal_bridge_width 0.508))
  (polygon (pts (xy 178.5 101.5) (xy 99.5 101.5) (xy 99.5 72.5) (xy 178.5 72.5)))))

